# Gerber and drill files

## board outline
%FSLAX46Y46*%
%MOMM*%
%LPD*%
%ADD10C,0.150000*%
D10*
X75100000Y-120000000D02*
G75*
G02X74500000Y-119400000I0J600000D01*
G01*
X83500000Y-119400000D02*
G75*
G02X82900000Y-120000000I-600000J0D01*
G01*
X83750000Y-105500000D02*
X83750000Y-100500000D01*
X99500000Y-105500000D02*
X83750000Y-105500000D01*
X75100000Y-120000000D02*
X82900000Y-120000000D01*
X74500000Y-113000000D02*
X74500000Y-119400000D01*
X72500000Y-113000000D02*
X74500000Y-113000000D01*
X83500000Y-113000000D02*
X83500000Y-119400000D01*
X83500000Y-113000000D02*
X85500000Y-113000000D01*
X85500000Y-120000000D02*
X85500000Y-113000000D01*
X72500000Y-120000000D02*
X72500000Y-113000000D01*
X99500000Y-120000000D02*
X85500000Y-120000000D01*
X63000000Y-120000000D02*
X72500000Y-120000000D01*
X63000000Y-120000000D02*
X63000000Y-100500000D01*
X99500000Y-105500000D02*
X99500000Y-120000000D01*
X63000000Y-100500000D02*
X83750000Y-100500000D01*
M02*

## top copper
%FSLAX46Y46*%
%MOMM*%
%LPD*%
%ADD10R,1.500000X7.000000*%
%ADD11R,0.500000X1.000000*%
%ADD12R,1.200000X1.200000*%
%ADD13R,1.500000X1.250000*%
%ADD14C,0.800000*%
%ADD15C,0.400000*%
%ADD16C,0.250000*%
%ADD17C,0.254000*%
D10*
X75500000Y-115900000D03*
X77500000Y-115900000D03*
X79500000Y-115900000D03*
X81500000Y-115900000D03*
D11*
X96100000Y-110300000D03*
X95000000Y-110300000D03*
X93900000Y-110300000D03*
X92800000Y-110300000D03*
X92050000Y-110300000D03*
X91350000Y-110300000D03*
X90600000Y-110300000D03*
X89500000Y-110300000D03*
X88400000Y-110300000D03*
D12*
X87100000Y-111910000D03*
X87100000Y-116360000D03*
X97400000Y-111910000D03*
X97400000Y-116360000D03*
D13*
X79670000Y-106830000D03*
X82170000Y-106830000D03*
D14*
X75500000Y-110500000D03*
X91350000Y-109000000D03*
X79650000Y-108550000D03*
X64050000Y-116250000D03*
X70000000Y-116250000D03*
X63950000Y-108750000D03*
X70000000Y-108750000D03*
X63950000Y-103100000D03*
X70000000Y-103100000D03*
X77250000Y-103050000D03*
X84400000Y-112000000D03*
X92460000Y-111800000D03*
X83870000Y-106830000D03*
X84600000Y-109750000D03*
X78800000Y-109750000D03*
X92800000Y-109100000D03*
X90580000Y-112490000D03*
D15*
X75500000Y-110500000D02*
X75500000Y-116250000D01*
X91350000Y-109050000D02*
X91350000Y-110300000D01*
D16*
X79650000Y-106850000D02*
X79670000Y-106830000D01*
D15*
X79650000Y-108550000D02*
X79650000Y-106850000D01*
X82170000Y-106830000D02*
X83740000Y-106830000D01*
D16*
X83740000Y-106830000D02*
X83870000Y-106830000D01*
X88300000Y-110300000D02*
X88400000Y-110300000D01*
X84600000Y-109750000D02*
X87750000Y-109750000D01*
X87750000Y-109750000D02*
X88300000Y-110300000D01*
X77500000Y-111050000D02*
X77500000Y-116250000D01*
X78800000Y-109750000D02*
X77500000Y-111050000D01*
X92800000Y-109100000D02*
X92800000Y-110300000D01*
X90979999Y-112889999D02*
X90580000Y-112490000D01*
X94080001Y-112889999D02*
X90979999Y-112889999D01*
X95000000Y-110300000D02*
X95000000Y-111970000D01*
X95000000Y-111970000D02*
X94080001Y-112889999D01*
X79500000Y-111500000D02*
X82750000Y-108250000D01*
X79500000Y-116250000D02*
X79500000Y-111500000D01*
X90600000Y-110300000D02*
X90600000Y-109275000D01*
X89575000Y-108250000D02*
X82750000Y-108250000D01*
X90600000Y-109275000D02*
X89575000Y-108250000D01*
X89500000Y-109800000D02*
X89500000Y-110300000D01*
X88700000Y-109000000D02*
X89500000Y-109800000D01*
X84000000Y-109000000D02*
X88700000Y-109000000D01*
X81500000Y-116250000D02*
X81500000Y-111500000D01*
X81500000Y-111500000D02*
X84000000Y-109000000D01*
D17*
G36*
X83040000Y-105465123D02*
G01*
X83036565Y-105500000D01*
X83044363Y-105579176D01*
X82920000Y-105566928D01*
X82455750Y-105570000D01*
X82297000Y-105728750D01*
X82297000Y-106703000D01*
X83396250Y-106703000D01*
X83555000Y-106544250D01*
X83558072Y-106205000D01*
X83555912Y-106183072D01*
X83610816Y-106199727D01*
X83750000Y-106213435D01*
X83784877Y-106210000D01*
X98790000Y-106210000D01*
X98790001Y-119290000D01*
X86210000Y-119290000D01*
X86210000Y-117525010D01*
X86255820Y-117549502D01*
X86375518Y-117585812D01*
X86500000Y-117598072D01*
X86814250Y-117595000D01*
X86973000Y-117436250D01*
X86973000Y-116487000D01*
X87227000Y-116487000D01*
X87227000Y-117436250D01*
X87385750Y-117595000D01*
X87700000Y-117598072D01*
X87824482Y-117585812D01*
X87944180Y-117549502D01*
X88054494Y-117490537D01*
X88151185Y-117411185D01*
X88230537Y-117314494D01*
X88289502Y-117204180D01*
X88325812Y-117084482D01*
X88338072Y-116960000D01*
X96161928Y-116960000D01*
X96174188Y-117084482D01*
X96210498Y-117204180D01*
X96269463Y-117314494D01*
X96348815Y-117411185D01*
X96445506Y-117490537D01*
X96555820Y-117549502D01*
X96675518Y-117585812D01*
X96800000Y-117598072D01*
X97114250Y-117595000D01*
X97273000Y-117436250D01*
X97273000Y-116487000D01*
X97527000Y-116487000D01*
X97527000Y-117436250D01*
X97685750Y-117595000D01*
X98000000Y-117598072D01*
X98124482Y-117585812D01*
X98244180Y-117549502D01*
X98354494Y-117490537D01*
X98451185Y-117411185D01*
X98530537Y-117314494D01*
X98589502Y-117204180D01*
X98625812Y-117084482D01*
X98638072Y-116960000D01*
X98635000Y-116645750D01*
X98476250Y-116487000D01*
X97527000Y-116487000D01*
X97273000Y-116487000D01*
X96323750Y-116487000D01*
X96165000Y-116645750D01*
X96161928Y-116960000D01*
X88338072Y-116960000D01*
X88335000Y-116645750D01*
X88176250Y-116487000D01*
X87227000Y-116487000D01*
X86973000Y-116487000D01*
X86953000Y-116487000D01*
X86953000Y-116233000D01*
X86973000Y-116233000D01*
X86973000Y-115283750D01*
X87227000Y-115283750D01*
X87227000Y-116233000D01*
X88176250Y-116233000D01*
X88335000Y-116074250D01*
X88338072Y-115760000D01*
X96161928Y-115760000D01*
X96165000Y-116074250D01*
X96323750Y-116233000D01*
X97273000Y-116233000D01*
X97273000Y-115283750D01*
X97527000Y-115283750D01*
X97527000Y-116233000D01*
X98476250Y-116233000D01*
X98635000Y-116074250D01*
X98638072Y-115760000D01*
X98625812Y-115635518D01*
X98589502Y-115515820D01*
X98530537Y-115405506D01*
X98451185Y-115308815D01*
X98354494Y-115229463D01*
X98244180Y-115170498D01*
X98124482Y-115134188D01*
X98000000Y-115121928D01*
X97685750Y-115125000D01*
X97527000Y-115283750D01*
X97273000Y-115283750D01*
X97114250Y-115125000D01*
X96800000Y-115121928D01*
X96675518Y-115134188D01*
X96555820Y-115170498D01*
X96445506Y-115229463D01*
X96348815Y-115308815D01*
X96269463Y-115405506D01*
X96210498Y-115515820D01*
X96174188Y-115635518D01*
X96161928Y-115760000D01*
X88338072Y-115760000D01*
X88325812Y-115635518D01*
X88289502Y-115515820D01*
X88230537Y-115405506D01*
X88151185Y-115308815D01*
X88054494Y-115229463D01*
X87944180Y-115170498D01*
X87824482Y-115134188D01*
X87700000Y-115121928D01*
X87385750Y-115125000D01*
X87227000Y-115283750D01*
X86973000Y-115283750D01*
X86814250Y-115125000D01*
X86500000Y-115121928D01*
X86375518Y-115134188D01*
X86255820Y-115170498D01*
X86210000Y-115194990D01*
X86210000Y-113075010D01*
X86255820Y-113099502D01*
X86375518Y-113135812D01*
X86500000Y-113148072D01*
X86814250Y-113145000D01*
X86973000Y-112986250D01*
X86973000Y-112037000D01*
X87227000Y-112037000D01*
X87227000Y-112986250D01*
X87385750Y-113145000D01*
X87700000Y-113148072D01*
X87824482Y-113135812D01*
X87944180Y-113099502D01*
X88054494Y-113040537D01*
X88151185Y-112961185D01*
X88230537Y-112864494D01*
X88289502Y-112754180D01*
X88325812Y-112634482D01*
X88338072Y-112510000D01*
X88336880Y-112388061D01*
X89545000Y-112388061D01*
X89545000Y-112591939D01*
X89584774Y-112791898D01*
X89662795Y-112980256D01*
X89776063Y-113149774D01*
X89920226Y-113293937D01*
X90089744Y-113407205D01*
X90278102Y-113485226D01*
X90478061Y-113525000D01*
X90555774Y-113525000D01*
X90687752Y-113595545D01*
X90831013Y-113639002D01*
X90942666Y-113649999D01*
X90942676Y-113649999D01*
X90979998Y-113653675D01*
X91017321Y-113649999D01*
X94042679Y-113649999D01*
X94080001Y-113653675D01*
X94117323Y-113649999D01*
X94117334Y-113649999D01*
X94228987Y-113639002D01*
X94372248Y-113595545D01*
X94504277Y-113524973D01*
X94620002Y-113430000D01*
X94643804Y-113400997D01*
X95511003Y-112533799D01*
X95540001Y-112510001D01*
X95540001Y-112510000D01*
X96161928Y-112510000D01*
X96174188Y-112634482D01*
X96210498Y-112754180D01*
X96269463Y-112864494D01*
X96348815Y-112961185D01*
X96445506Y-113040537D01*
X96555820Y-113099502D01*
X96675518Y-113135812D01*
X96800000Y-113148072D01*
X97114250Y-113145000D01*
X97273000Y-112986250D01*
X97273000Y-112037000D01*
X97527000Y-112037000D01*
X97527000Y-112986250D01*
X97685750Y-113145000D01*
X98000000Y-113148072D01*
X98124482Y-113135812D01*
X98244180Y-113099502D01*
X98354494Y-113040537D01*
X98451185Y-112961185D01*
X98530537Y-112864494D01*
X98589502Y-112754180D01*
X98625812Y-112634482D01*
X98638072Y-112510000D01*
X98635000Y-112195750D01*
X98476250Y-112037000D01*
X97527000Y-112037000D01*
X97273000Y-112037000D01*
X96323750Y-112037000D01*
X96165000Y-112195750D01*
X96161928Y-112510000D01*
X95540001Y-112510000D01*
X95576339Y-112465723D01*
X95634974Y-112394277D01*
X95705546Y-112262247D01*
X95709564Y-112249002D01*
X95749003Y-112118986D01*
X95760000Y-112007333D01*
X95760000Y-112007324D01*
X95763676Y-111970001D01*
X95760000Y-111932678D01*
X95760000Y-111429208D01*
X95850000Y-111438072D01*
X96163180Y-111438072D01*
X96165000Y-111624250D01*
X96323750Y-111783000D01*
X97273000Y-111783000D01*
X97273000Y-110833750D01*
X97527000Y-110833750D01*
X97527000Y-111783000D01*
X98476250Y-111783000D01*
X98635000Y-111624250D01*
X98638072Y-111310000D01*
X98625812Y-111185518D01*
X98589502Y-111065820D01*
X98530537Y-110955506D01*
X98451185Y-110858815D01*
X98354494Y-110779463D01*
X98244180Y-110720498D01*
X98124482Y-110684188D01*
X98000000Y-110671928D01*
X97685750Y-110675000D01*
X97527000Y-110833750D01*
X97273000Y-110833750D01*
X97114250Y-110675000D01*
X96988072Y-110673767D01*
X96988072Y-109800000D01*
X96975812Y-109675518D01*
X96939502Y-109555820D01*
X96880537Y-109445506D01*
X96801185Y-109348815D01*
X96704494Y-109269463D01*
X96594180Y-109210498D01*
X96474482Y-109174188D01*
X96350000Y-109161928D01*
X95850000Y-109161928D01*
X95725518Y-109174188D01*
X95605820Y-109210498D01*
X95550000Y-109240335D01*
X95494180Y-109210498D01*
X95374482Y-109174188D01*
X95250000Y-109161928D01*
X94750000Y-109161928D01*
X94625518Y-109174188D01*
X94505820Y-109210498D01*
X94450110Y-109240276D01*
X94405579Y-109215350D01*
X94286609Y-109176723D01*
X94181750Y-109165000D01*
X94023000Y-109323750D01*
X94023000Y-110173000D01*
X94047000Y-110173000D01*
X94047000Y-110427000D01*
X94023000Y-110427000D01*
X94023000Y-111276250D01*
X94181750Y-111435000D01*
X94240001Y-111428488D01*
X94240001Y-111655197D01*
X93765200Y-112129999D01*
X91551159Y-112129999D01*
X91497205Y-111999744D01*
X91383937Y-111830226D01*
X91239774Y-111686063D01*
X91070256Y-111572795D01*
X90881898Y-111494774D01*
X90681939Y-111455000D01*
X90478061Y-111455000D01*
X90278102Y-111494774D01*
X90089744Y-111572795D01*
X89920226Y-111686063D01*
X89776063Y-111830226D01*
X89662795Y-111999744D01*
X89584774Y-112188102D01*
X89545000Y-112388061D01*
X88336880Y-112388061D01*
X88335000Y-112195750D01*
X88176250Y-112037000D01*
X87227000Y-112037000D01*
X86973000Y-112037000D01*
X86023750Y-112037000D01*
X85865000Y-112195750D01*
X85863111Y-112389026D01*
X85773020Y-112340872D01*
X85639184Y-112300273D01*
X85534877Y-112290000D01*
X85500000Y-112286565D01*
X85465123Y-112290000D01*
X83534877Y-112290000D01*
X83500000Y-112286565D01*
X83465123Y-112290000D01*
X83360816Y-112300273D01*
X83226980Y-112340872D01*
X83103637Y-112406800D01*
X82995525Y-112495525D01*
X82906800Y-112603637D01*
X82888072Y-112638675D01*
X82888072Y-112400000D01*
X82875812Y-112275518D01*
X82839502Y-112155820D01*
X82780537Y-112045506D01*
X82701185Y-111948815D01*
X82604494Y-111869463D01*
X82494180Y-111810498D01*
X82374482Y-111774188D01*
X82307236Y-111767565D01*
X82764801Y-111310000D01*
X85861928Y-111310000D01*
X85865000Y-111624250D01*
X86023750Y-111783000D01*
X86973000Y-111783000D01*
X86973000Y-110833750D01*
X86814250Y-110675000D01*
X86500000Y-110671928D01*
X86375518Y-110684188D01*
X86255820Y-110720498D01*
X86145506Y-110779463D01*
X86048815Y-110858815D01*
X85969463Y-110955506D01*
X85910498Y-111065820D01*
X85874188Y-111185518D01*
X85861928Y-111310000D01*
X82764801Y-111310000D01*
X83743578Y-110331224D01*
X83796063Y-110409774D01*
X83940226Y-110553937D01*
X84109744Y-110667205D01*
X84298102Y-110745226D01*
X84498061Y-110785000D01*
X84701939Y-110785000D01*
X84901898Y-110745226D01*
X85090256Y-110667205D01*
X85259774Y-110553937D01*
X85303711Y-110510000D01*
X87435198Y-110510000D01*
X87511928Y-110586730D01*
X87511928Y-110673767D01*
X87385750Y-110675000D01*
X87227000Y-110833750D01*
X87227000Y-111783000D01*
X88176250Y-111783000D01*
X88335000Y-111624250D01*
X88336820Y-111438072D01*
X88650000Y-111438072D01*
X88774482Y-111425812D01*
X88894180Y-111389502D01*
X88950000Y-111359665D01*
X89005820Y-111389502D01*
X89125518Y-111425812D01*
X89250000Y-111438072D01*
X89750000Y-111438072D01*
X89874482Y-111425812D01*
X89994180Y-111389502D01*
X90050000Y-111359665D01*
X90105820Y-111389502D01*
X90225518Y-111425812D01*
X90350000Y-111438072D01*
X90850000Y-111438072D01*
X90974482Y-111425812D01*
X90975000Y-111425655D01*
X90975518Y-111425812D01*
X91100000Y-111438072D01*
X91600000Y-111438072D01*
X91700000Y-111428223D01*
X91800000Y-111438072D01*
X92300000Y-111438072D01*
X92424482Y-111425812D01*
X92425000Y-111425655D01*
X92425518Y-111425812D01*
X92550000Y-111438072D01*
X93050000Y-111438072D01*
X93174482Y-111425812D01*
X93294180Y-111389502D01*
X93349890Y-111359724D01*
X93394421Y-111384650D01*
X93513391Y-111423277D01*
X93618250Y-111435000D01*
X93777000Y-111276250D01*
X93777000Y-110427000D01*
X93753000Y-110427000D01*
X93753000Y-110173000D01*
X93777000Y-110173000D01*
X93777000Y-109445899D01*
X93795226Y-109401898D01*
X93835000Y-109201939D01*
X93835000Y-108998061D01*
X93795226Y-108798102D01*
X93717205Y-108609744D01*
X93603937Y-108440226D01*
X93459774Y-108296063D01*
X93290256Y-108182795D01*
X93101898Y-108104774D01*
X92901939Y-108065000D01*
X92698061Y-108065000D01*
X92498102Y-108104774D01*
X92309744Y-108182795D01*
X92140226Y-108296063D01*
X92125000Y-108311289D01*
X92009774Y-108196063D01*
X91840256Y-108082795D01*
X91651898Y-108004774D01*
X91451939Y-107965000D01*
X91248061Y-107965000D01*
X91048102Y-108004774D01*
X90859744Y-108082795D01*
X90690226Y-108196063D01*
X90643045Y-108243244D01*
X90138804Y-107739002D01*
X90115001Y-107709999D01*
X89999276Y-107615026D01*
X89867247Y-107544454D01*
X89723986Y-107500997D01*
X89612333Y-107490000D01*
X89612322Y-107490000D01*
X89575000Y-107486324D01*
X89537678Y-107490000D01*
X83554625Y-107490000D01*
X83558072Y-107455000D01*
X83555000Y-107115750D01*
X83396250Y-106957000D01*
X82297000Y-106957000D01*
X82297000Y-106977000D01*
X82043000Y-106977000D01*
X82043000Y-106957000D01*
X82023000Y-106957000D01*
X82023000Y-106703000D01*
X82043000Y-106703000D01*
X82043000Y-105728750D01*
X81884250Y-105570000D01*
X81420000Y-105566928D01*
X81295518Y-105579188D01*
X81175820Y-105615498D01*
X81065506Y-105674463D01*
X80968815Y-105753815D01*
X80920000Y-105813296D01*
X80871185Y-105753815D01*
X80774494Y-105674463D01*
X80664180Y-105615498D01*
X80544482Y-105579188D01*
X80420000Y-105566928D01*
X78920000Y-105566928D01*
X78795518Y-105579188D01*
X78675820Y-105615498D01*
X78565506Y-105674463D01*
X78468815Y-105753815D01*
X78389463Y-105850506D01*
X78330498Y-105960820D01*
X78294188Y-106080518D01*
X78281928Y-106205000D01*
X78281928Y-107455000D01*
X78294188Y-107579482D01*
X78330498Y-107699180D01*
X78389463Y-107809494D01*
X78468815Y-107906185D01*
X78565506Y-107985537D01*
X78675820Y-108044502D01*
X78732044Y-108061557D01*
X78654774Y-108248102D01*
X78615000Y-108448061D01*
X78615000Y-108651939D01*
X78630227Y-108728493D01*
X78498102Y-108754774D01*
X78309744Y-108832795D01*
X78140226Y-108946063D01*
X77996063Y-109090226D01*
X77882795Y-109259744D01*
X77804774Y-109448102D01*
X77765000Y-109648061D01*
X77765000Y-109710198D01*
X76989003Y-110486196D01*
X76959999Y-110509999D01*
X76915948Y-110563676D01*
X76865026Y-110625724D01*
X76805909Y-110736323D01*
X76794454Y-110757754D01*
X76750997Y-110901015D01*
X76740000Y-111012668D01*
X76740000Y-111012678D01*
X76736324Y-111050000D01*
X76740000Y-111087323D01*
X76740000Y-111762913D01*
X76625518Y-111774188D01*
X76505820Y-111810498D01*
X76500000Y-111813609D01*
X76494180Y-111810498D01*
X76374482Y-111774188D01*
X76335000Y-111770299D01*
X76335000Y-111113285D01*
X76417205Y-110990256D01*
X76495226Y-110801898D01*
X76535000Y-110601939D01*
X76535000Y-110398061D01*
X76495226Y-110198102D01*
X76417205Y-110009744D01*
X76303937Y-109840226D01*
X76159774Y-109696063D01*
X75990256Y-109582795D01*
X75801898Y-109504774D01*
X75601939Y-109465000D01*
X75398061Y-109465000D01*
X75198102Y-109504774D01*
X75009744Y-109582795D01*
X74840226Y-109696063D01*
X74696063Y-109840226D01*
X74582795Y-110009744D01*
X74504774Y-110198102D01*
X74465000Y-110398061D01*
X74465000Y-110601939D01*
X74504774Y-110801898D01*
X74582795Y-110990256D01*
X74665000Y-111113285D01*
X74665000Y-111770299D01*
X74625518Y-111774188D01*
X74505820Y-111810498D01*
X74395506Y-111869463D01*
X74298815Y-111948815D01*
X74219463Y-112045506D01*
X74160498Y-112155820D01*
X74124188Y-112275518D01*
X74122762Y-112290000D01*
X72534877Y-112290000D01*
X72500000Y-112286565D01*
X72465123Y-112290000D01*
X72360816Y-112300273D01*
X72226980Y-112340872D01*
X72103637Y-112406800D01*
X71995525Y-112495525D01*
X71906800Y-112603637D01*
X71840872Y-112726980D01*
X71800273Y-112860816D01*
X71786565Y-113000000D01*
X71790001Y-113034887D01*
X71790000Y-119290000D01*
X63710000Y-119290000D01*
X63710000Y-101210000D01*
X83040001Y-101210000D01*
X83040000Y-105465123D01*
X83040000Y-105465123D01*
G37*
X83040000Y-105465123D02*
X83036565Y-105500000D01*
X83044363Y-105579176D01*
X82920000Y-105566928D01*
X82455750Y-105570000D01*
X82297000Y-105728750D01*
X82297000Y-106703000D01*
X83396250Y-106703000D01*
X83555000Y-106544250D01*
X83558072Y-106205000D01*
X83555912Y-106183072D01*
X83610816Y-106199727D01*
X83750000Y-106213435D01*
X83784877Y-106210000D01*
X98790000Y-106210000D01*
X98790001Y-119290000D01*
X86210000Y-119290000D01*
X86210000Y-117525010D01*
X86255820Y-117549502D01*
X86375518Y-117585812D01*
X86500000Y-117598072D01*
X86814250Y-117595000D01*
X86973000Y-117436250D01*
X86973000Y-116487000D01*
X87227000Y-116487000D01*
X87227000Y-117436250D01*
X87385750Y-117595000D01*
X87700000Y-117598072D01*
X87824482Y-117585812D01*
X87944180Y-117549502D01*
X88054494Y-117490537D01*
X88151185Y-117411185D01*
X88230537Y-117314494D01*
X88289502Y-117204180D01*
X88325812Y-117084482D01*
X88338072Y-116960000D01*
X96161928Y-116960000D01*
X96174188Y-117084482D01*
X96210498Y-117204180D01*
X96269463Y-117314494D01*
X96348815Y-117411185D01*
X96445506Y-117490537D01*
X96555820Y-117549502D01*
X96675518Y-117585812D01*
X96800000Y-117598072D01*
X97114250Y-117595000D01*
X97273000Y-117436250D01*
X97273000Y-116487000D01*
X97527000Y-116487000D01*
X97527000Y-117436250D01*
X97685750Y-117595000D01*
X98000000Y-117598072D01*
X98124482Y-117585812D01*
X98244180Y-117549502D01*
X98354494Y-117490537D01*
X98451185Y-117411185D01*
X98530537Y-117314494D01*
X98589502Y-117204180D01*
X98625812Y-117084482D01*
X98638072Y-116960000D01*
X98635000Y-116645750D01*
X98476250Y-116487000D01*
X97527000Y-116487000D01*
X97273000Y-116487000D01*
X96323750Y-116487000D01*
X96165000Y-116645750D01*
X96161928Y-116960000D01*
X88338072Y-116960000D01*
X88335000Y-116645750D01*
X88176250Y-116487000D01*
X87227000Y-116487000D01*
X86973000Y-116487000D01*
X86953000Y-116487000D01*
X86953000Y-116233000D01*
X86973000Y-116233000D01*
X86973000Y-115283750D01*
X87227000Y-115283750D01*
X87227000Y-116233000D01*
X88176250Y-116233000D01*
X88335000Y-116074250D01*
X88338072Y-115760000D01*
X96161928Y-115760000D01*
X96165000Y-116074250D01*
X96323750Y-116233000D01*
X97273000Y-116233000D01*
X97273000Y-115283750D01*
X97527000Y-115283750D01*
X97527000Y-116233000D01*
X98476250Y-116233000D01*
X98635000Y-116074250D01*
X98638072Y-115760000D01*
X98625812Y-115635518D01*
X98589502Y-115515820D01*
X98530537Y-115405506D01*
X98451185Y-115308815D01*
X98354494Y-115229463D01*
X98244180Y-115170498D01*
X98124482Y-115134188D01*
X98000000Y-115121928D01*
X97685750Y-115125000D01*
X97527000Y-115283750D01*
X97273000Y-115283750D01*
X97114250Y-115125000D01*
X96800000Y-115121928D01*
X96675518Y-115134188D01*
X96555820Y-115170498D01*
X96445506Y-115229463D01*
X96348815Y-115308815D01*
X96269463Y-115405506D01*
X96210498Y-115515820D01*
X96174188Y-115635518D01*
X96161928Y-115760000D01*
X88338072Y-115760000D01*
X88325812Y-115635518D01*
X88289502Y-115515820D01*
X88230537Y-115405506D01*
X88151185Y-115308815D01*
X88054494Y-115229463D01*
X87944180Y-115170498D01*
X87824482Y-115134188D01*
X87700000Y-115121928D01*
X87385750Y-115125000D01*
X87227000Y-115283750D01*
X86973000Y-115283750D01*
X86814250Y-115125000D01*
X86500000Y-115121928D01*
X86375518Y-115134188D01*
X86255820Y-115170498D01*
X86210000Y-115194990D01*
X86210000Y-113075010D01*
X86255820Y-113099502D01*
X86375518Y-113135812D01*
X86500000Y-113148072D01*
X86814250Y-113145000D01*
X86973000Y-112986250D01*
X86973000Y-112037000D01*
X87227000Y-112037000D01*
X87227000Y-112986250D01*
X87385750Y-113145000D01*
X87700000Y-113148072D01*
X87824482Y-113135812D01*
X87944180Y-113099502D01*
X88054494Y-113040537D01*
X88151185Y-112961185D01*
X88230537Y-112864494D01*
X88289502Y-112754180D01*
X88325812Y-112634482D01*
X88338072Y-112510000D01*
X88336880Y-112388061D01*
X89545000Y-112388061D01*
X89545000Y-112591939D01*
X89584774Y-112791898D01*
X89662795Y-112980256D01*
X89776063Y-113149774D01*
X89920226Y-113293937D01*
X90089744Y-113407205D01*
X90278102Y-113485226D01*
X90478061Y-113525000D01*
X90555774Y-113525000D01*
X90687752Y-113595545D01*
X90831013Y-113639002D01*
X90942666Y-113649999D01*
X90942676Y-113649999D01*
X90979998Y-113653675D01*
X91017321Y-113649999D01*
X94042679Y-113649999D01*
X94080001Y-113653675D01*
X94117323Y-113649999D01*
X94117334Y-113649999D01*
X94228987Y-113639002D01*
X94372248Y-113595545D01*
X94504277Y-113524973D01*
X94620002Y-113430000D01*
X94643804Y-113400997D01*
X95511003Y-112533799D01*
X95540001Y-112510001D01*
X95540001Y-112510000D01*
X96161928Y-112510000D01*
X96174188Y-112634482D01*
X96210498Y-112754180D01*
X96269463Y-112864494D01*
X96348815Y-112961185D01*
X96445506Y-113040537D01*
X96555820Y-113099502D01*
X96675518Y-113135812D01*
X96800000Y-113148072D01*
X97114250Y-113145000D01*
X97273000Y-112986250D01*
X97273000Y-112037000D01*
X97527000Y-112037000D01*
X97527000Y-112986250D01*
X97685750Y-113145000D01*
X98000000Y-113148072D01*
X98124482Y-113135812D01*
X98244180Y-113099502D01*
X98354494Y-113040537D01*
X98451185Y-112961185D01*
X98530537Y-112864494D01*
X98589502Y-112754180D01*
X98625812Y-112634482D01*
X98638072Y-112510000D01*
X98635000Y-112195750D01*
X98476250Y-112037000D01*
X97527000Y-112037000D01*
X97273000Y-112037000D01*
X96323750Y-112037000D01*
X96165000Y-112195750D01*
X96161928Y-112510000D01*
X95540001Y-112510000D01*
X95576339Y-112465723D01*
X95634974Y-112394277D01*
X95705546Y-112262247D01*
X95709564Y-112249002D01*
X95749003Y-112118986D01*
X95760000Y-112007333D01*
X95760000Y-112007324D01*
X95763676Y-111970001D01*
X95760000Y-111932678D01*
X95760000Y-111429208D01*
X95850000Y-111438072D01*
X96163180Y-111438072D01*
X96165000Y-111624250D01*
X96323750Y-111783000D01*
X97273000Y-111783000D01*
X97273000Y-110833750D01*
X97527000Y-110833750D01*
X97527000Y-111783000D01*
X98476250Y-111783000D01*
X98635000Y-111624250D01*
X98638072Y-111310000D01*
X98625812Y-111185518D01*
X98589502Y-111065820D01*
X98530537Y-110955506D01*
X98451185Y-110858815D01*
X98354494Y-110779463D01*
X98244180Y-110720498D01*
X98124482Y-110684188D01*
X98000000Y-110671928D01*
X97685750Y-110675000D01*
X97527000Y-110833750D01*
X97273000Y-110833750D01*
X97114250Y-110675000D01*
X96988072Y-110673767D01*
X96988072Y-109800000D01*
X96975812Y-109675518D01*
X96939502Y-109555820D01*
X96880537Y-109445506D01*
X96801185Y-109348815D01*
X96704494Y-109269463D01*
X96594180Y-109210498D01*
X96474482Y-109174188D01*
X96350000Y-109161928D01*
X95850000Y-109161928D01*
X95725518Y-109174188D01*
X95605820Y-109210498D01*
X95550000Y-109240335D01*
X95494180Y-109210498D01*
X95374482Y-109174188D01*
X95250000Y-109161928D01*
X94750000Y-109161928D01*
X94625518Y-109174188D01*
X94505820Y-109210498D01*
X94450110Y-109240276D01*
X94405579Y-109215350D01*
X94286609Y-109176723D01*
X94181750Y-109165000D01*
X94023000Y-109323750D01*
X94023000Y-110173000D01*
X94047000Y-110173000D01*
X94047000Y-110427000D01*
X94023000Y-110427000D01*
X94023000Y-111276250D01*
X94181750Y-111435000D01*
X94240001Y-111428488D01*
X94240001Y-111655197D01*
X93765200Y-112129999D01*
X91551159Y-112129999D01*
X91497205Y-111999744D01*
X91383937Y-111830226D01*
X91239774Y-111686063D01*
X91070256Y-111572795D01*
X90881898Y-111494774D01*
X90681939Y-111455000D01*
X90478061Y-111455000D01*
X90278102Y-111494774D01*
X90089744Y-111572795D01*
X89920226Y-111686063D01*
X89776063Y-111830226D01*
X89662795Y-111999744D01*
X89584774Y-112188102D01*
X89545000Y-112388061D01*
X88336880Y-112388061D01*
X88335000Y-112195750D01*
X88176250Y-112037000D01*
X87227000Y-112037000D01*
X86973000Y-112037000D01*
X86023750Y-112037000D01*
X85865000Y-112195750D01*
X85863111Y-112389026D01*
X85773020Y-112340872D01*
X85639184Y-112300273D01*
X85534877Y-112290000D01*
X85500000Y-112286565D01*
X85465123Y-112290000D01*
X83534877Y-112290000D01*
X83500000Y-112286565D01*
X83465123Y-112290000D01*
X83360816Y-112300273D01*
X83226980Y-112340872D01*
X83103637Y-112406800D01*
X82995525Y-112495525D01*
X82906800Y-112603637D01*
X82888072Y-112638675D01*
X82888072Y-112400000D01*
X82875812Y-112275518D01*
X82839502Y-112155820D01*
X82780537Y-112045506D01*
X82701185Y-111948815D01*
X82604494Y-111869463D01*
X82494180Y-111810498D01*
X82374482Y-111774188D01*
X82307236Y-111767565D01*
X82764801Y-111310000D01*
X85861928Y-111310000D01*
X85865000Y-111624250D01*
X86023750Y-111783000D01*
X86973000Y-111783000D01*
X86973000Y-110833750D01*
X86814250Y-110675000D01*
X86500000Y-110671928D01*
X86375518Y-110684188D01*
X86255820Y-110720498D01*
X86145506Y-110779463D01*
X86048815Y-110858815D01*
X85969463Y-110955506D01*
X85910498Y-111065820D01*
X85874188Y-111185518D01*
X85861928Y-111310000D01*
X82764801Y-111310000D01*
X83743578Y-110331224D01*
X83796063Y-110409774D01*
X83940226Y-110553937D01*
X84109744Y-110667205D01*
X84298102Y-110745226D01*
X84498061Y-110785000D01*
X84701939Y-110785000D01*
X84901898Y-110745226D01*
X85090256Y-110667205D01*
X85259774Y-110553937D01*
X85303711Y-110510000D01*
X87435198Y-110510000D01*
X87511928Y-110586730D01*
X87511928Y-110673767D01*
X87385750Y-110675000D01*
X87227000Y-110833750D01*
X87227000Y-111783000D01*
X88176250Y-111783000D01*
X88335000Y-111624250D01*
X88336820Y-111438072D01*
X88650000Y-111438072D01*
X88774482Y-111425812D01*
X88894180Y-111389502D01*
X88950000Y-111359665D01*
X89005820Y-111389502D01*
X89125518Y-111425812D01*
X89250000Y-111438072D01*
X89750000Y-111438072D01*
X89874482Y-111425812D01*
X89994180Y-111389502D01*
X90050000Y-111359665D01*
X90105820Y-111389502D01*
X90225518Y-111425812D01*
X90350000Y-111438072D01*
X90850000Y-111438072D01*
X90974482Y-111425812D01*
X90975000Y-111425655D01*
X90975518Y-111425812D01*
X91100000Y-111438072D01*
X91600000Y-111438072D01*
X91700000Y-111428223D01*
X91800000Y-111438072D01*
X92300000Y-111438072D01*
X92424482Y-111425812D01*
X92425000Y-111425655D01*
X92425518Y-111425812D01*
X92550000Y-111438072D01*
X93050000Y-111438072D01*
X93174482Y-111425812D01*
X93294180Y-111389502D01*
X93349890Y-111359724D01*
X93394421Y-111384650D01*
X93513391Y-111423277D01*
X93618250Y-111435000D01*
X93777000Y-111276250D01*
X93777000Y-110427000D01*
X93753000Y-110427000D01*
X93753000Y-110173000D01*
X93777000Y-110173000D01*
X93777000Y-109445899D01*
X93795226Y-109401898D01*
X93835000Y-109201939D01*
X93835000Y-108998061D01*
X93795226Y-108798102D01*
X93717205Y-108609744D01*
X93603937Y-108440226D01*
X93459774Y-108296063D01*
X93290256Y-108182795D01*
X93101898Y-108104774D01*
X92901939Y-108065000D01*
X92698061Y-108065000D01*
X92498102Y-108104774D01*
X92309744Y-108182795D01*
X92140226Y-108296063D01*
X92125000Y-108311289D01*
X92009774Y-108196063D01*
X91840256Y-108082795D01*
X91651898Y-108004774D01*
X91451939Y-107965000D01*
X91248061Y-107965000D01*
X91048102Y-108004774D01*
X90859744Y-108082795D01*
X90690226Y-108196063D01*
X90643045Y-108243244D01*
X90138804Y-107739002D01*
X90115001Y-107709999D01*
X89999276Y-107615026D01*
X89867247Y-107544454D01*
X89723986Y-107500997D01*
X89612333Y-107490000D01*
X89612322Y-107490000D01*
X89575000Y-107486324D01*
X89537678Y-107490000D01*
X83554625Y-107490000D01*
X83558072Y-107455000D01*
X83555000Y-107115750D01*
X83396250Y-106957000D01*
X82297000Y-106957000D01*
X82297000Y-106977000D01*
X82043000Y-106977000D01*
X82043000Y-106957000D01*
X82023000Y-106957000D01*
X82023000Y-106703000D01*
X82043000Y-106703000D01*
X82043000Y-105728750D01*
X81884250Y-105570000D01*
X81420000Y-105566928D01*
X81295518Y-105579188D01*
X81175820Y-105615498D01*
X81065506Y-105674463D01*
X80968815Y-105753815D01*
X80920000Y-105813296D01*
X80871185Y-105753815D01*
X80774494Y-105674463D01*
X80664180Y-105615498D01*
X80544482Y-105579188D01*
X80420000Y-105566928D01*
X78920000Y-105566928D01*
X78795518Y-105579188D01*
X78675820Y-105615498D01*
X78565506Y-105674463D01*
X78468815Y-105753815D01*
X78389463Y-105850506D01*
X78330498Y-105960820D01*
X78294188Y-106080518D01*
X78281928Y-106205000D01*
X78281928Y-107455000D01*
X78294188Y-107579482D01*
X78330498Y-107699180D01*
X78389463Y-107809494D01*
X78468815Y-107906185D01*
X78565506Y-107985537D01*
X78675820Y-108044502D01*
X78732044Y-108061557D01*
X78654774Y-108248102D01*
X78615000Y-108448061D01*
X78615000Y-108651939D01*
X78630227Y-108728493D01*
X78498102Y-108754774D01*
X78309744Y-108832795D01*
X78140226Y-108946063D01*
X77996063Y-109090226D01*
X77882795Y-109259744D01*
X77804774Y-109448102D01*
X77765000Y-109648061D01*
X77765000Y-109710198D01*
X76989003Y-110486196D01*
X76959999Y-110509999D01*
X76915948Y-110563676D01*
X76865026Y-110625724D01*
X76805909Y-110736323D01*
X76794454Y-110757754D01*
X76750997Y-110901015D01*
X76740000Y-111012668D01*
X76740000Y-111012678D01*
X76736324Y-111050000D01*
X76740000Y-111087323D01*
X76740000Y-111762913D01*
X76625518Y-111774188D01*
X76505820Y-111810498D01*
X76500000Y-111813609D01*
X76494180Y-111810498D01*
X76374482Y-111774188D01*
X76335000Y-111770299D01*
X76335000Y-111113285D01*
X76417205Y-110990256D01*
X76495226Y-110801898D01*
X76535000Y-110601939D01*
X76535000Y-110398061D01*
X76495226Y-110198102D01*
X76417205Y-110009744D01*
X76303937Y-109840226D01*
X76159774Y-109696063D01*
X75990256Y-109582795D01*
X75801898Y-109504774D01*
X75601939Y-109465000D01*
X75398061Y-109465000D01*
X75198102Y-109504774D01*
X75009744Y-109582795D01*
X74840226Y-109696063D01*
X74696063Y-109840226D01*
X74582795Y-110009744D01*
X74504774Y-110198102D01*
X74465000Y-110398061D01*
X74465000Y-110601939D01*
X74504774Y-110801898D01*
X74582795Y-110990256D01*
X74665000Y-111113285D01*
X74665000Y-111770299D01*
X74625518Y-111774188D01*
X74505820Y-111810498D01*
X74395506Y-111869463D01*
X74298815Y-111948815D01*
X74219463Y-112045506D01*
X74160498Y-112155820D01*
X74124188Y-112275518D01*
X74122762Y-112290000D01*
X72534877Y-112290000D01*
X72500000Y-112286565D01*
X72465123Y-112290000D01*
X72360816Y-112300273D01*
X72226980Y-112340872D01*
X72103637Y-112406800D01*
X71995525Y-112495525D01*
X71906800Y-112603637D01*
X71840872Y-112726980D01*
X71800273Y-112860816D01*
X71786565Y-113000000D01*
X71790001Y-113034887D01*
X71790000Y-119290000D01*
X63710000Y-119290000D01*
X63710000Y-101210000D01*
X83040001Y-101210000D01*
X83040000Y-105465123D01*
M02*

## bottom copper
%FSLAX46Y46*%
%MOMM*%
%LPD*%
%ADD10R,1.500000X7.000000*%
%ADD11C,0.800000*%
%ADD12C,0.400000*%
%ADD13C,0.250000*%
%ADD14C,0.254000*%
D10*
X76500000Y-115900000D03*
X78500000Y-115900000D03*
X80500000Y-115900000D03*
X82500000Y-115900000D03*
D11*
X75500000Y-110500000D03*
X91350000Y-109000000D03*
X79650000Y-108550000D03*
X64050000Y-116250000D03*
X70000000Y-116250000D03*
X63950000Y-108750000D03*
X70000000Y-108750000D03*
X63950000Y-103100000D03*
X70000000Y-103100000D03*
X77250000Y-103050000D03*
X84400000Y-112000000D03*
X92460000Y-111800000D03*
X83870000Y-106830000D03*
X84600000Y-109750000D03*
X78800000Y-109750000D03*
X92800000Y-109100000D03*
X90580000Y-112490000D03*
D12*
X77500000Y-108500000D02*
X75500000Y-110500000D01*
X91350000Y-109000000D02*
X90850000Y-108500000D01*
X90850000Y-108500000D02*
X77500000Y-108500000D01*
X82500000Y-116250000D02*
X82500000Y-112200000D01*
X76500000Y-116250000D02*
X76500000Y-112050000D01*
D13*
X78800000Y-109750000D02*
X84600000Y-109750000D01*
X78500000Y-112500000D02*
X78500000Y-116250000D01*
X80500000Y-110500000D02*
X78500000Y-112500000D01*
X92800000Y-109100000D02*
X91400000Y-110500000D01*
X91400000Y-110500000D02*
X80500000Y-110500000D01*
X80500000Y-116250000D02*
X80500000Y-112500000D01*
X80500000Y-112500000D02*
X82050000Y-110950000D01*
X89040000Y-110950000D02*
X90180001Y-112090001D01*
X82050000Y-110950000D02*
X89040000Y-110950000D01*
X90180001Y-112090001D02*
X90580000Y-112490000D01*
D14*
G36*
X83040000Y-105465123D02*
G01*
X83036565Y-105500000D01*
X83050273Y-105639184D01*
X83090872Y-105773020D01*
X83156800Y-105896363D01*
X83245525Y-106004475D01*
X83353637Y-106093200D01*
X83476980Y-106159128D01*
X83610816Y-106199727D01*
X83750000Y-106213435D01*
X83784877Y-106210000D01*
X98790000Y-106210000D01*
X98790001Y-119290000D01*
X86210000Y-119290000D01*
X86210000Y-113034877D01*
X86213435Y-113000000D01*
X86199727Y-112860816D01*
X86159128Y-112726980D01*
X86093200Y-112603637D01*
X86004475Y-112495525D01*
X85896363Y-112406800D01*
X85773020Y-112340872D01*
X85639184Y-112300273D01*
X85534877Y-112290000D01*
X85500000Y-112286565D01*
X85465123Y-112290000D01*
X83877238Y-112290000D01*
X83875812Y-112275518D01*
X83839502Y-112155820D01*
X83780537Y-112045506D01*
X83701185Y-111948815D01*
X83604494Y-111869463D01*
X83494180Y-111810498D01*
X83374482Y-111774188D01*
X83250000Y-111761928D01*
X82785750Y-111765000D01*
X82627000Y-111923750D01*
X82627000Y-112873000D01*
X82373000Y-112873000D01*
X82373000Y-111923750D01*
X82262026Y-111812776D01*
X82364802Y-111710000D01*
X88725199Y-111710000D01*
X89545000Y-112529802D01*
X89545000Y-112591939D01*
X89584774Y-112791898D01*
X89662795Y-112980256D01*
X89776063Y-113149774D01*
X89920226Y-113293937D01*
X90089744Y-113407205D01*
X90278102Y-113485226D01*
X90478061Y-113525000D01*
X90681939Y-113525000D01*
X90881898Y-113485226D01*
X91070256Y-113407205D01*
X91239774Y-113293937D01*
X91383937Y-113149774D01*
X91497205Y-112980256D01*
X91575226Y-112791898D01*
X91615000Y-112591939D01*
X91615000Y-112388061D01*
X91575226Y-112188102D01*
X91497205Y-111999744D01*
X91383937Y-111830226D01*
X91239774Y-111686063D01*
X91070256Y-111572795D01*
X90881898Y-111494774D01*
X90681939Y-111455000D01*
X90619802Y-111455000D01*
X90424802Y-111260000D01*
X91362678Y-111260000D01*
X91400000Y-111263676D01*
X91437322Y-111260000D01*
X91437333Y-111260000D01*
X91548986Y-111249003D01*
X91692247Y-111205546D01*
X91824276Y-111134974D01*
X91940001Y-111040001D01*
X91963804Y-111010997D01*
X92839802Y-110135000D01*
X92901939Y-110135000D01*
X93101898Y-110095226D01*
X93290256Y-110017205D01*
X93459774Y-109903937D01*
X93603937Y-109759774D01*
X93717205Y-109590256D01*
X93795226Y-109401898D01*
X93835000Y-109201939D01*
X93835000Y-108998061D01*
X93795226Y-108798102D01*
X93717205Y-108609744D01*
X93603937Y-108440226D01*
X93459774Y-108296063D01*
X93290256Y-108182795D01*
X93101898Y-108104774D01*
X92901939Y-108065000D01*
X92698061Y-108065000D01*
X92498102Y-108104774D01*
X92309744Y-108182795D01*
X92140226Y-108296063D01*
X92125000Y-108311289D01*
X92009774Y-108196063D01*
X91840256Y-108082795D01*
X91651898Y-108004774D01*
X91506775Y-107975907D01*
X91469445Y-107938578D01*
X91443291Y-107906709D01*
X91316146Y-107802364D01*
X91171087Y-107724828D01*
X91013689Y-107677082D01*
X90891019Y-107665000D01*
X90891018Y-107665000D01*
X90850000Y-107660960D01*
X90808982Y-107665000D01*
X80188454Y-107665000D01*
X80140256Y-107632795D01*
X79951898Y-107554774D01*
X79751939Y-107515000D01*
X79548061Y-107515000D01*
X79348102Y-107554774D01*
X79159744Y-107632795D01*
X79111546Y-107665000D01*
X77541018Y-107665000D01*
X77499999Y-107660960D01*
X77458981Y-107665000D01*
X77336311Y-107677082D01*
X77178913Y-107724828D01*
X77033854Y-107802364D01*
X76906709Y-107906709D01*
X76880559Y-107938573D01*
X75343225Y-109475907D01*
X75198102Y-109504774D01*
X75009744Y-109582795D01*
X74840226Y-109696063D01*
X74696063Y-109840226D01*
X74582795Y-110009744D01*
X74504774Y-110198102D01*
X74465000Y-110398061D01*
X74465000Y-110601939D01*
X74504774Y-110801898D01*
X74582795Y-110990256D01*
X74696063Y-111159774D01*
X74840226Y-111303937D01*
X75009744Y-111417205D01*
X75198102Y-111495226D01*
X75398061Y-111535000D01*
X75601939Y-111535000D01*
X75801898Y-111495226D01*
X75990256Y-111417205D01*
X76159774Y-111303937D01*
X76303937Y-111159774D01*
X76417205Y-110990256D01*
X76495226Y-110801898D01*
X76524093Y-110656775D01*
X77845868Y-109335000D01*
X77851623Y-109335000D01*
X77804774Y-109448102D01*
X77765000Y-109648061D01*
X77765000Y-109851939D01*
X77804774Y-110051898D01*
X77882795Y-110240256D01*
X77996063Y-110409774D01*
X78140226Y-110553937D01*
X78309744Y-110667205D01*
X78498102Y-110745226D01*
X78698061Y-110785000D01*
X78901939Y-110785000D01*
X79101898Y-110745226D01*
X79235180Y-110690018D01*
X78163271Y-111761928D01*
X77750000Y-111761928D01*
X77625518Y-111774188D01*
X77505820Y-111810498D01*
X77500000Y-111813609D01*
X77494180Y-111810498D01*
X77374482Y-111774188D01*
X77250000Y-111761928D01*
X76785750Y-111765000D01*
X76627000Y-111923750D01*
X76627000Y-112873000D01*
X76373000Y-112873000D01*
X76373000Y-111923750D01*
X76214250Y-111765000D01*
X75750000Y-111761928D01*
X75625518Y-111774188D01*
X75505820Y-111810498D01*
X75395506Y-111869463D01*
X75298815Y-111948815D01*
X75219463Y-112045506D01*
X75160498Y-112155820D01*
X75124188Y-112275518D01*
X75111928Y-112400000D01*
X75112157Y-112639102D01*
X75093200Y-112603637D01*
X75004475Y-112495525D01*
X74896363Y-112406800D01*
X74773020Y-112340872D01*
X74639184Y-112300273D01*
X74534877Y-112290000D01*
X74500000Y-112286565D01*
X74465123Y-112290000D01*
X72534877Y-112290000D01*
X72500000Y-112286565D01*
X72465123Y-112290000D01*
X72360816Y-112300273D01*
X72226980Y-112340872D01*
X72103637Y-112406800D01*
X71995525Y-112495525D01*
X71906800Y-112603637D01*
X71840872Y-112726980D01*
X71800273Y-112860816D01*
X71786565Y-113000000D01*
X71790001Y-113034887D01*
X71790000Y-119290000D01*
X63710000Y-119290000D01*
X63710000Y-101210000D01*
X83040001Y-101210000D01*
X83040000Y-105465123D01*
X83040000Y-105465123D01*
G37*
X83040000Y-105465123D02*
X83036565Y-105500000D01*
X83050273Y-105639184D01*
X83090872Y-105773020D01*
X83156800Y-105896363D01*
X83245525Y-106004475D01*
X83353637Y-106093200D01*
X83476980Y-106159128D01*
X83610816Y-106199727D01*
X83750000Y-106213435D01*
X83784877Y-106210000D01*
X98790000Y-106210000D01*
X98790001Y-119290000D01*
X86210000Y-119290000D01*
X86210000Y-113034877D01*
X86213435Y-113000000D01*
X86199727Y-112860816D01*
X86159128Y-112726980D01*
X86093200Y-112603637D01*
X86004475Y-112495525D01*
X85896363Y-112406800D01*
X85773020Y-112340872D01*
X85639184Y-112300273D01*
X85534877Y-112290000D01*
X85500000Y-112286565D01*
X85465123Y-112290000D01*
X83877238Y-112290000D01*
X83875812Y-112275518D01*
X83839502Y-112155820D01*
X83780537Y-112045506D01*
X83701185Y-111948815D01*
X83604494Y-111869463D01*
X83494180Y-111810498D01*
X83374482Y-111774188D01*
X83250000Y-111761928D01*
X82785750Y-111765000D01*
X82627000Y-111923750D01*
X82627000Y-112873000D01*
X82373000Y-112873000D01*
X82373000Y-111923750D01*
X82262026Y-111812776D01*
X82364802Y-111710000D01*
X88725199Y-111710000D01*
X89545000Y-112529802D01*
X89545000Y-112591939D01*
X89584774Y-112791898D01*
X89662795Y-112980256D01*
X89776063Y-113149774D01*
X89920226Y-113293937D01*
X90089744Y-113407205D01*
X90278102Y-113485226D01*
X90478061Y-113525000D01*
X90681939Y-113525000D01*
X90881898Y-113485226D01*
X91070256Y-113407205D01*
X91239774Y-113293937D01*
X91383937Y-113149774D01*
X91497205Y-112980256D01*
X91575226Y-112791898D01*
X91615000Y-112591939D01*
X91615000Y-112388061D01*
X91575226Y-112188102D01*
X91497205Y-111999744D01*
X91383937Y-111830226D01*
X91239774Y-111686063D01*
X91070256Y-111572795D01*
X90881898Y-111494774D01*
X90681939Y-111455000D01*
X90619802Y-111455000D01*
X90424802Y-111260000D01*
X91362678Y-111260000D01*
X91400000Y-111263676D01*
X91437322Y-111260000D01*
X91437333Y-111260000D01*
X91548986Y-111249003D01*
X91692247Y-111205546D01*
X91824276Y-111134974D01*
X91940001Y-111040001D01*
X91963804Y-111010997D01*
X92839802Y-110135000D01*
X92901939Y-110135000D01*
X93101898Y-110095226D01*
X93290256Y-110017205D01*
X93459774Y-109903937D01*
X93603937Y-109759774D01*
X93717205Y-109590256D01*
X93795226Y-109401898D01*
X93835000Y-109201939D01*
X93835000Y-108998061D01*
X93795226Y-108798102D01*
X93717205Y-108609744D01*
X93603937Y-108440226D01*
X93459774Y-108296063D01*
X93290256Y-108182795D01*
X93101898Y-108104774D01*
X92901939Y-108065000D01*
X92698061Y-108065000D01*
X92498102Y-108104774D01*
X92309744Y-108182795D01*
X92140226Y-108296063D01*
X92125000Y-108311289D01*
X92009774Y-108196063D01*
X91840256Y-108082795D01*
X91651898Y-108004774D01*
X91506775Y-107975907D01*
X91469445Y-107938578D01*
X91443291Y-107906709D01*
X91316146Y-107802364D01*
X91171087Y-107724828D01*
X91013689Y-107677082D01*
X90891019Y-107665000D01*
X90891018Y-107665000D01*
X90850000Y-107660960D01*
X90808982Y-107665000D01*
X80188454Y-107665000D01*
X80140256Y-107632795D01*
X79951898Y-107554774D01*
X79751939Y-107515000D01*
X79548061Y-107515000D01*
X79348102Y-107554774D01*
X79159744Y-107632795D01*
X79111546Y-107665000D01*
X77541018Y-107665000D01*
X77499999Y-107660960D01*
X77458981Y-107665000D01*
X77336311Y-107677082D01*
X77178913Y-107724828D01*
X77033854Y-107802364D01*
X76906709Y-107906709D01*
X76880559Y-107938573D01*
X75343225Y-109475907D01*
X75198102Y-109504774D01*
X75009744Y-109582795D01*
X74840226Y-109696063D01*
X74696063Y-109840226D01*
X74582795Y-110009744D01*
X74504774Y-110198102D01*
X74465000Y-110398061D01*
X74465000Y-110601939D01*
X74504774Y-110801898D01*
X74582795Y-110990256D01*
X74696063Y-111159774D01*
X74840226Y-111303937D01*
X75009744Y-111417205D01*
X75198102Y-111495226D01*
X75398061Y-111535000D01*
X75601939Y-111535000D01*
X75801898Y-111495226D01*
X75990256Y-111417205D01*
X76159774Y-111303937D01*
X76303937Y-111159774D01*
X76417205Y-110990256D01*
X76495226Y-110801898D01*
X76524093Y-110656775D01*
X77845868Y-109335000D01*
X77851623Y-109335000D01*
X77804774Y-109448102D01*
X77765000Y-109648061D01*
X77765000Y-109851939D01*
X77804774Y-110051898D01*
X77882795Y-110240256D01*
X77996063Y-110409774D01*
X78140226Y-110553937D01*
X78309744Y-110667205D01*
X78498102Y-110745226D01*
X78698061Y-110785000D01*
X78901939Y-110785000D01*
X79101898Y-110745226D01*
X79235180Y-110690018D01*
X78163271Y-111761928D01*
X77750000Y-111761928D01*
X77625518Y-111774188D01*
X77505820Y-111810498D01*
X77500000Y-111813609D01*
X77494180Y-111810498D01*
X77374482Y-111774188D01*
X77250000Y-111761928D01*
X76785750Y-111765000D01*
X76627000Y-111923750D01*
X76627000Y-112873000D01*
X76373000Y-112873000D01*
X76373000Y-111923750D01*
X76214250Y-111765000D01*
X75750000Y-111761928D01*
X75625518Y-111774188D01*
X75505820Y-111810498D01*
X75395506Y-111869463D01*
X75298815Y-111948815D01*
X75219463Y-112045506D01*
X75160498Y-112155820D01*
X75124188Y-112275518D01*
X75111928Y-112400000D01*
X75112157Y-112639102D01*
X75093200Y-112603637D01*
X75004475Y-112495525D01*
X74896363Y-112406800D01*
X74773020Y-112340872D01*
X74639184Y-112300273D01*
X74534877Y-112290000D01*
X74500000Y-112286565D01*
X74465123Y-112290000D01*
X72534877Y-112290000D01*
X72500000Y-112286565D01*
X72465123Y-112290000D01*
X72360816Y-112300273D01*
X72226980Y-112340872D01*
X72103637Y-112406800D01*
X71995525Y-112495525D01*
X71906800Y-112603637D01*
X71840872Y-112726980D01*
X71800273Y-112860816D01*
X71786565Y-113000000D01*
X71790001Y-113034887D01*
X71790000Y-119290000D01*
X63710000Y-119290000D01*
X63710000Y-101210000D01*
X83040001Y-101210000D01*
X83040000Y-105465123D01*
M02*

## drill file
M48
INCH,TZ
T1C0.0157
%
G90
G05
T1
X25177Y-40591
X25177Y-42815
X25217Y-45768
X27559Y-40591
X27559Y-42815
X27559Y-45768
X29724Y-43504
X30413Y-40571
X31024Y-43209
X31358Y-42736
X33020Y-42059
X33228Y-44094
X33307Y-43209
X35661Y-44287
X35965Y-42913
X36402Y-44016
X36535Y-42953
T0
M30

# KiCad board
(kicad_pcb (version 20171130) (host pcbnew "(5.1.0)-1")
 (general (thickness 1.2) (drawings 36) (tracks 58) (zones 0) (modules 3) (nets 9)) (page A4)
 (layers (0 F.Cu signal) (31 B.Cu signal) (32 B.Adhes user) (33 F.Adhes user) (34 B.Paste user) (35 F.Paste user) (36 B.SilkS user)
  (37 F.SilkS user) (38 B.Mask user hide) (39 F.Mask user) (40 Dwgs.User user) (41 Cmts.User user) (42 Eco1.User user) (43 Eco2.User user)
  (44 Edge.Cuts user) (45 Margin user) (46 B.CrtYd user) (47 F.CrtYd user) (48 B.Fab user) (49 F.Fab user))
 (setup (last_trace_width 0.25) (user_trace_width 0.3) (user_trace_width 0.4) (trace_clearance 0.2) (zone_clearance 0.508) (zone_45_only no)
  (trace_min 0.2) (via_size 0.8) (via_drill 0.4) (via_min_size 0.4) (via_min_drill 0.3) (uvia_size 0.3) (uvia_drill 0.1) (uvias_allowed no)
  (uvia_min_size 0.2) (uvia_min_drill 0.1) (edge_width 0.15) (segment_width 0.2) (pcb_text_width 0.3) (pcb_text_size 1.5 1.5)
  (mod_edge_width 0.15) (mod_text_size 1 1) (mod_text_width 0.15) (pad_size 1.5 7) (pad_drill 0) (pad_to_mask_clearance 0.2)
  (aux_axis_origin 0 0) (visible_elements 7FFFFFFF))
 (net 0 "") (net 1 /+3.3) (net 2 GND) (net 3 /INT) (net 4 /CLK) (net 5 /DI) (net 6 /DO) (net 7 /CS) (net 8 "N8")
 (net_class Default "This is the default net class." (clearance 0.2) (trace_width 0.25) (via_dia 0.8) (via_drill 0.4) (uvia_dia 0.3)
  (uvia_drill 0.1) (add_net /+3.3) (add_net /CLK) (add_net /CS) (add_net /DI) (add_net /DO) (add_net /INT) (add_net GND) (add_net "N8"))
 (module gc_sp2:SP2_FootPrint (layer F.Cu) (at 75.5 115.9)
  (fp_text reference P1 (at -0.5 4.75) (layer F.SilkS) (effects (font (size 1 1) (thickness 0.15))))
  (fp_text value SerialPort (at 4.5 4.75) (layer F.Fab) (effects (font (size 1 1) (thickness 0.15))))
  (pad 1 smd rect (at 0 0) (size 1.5 7) (layers F.Cu F.Paste F.Mask) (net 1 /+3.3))
  (pad 2 smd rect (at 1 0) (size 1.5 7) (layers B.Cu B.Paste B.Mask) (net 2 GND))
  (pad 3 smd rect (at 2 0) (size 1.5 7) (layers F.Cu F.Paste F.Mask) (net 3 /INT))
  (pad 4 smd rect (at 3 0) (size 1.5 7) (layers B.Cu B.Adhes B.Mask) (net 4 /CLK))
  (pad 5 smd rect (at 4 0) (size 1.5 7) (layers F.Cu F.Paste F.Mask) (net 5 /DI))
  (pad 6 smd rect (at 5 0) (size 1.5 7) (layers B.Cu B.Paste B.Mask) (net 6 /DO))
  (pad 7 smd rect (at 6 0) (size 1.5 7) (layers F.Cu F.Paste F.Mask) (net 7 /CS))
  (pad 8 smd rect (at 7 0) (size 1.5 7) (layers B.Cu B.Paste B.Mask) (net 2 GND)))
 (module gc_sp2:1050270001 (layer F.Cu) (at 96.1 110.3 180)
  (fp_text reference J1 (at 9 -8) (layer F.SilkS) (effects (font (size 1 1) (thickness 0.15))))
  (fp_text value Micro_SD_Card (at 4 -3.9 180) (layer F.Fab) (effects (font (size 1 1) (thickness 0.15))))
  (pad 8 smd rect (at 0 0 180) (size 0.5 1) (layers F.Cu F.Paste F.Mask) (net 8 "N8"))
  (pad 7 smd rect (at 1.1 0 180) (size 0.5 1) (layers F.Cu F.Paste F.Mask) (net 6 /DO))
  (pad 6 smd rect (at 2.2 0 180) (size 0.5 1) (layers F.Cu F.Paste F.Mask) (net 2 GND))
  (pad 5 smd rect (at 3.3 0 180) (size 0.5 1) (layers F.Cu F.Paste F.Mask) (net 4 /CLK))
  (pad "" smd rect (at 4.05 0 180) (size 0.5 1) (layers F.Cu F.Paste F.Mask))
  (pad 4 smd rect (at 4.75 0 180) (size 0.5 1) (layers F.Cu F.Paste F.Mask) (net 1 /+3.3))
  (pad 3 smd rect (at 5.5 0 180) (size 0.5 1) (layers F.Cu F.Paste F.Mask) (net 5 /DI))
  (pad 2 smd rect (at 6.6 0 180) (size 0.5 1) (layers F.Cu F.Paste F.Mask) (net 7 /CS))
  (pad 1 smd rect (at 7.7 0 180) (size 0.5 1) (layers F.Cu F.Paste F.Mask) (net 3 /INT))
  (pad 9 smd rect (at 9 -1.61 180) (size 1.2 1.2) (layers F.Cu F.Paste F.Mask) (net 2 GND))
  (pad 9 smd rect (at 9 -6.06 180) (size 1.2 1.2) (layers F.Cu F.Paste F.Mask) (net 2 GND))
  (pad 9 smd rect (at -1.3 -1.61 180) (size 1.2 1.2) (layers F.Cu F.Paste F.Mask) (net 2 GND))
  (pad 9 smd rect (at -1.3 -6.06 180) (size 1.2 1.2) (layers F.Cu F.Paste F.Mask) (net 2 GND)))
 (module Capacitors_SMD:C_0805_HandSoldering (layer F.Cu) (at 80.92 106.83)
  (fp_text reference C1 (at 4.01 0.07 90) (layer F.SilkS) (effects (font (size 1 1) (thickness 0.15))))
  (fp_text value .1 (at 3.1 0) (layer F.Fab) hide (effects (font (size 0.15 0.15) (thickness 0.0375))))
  (pad 1 smd rect (at -1.25 0) (size 1.5 1.25) (layers F.Cu F.Paste F.Mask) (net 1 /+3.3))
  (pad 2 smd rect (at 1.25 0) (size 1.5 1.25) (layers F.Cu F.Paste F.Mask) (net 2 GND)))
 (gr_arc (start 75.1 119.4) (end 74.5 119.4) (angle -90) (layer Edge.Cuts) (width 0.15))
 (gr_arc (start 82.9 119.4) (end 82.9 120) (angle -90) (layer Edge.Cuts) (width 0.15))
 (gr_line (start 83.75 105.5) (end 83.75 100.5) (layer Edge.Cuts) (width 0.15))
 (gr_line (start 99.5 105.5) (end 83.75 105.5) (layer Edge.Cuts) (width 0.15))
 (gr_line (start 75.1 120) (end 82.9 120) (layer Edge.Cuts) (width 0.15))
 (gr_line (start 74.5 113) (end 74.5 119.4) (layer Edge.Cuts) (width 0.15))
 (gr_line (start 72.5 113) (end 74.5 113) (layer Edge.Cuts) (width 0.15))
 (gr_line (start 83.5 113) (end 83.5 119.4) (layer Edge.Cuts) (width 0.15))
 (gr_line (start 83.5 113) (end 85.5 113) (layer Edge.Cuts) (width 0.15))
 (gr_line (start 85.5 120) (end 85.5 113) (layer Edge.Cuts) (width 0.15))
 (gr_line (start 72.5 120) (end 72.5 113) (layer Edge.Cuts) (width 0.15))
 (gr_line (start 99.5 120) (end 85.5 120) (layer Edge.Cuts) (width 0.15))
 (gr_line (start 63 120) (end 72.5 120) (layer Edge.Cuts) (width 0.15))
 (gr_line (start 63 120) (end 63 100.5) (layer Edge.Cuts) (width 0.15))
 (gr_line (start 99.5 105.5) (end 99.5 120) (layer Edge.Cuts) (width 0.15))
 (gr_line (start 63 100.5) (end 83.75 100.5) (layer Edge.Cuts) (width 0.15))
 (via (at 75.5 110.5) (size 0.8) (drill 0.4) (layers F.Cu B.Cu) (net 1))
 (segment (start 75.5 110.5) (end 75.5 116.25) (width 0.4) (layer F.Cu) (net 1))
 (segment (start 91.35 109.05) (end 91.35 110.3) (width 0.4) (layer F.Cu) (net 1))
 (via (at 91.35 109) (size 0.8) (drill 0.4) (layers F.Cu B.Cu) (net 1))
 (segment (start 77.5 108.5) (end 75.5 110.5) (width 0.4) (layer B.Cu) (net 1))
 (segment (start 91.35 109) (end 90.85 108.5) (width 0.4) (layer B.Cu) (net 1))
 (segment (start 90.85 108.5) (end 77.5 108.5) (width 0.4) (layer B.Cu) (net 1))
 (via (at 79.65 108.55) (size 0.8) (drill 0.4) (layers F.Cu B.Cu) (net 1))
 (segment (start 79.65 106.85) (end 79.67 106.83) (width 0.25) (layer F.Cu) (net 1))
 (segment (start 79.65 108.55) (end 79.65 106.85) (width 0.4) (layer F.Cu) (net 1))
 (via (at 64.05 116.25) (size 0.8) (drill 0.4) (layers F.Cu B.Cu) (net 2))
 (via (at 70 116.25) (size 0.8) (drill 0.4) (layers F.Cu B.Cu) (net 2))
 (via (at 63.95 108.75) (size 0.8) (drill 0.4) (layers F.Cu B.Cu) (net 2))
 (via (at 70 108.75) (size 0.8) (drill 0.4) (layers F.Cu B.Cu) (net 2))
 (via (at 63.95 103.1) (size 0.8) (drill 0.4) (layers F.Cu B.Cu) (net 2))
 (via (at 70 103.1) (size 0.8) (drill 0.4) (layers F.Cu B.Cu) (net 2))
 (via (at 77.25 103.05) (size 0.8) (drill 0.4) (layers F.Cu B.Cu) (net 2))
 (via (at 84.4 112) (size 0.8) (drill 0.4) (layers F.Cu B.Cu) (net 2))
 (segment (start 82.5 116.25) (end 82.5 112.2) (width 0.4) (layer B.Cu) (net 2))
 (segment (start 76.5 116.25) (end 76.5 112.05) (width 0.4) (layer B.Cu) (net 2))
 (via (at 92.46 111.8) (size 0.8) (drill 0.4) (layers F.Cu B.Cu) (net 2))
 (segment (start 82.17 106.83) (end 83.74 106.83) (width 0.4) (layer F.Cu) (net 2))
 (via (at 83.87 106.83) (size 0.8) (drill 0.4) (layers F.Cu B.Cu) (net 2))
 (segment (start 83.74 106.83) (end 83.87 106.83) (width 0.25) (layer F.Cu) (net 2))
 (via (at 84.6 109.75) (size 0.8) (drill 0.4) (layers F.Cu B.Cu) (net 3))
 (segment (start 88.3 110.3) (end 88.4 110.3) (width 0.25) (layer F.Cu) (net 3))
 (segment (start 84.6 109.75) (end 87.75 109.75) (width 0.25) (layer F.Cu) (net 3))
 (segment (start 87.75 109.75) (end 88.3 110.3) (width 0.25) (layer F.Cu) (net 3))
 (via (at 78.8 109.75) (size 0.8) (drill 0.4) (layers F.Cu B.Cu) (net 3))
 (segment (start 78.8 109.75) (end 84.6 109.75) (width 0.25) (layer B.Cu) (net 3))
 (segment (start 77.5 111.05) (end 77.5 116.25) (width 0.25) (layer F.Cu) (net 3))
 (segment (start 78.8 109.75) (end 77.5 111.05) (width 0.25) (layer F.Cu) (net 3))
 (via (at 92.8 109.1) (size 0.8) (drill 0.4) (layers F.Cu B.Cu) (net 4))
 (segment (start 92.8 109.1) (end 92.8 110.3) (width 0.25) (layer F.Cu) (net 4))
 (segment (start 78.5 112.5) (end 78.5 116.25) (width 0.25) (layer B.Cu) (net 4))
 (segment (start 80.5 110.5) (end 78.5 112.5) (width 0.25) (layer B.Cu) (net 4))
 (segment (start 92.8 109.1) (end 91.4 110.5) (width 0.25) (layer B.Cu) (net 4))
 (segment (start 91.4 110.5) (end 80.5 110.5) (width 0.25) (layer B.Cu) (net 4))
 (segment (start 80.5 116.25) (end 80.5 112.5) (width 0.25) (layer B.Cu) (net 6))
 (via (at 90.58 112.49) (size 0.8) (drill 0.4) (layers F.Cu B.Cu) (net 6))
 (segment (start 80.5 112.5) (end 82.05 110.95) (width 0.25) (layer B.Cu) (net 6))
 (segment (start 89.04 110.95) (end 90.180001 112.090001) (width 0.25) (layer B.Cu) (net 6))
 (segment (start 82.05 110.95) (end 89.04 110.95) (width 0.25) (layer B.Cu) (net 6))
 (segment (start 90.180001 112.090001) (end 90.58 112.49) (width 0.25) (layer B.Cu) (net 6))
 (segment (start 90.979999 112.889999) (end 90.58 112.49) (width 0.25) (layer F.Cu) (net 6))
 (segment (start 94.080001 112.889999) (end 90.979999 112.889999) (width 0.25) (layer F.Cu) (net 6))
 (segment (start 95 110.3) (end 95 111.97) (width 0.25) (layer F.Cu) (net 6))
 (segment (start 95 111.97) (end 94.080001 112.889999) (width 0.25) (layer F.Cu) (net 6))
 (segment (start 79.5 111.5) (end 82.75 108.25) (width 0.25) (layer F.Cu) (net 5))
 (segment (start 79.5 116.25) (end 79.5 111.5) (width 0.25) (layer F.Cu) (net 5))
 (segment (start 90.6 110.3) (end 90.6 109.275) (width 0.25) (layer F.Cu) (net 5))
 (segment (start 89.575 108.25) (end 82.75 108.25) (width 0.25) (layer F.Cu) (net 5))
 (segment (start 90.6 109.275) (end 89.575 108.25) (width 0.25) (layer F.Cu) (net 5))
 (segment (start 89.5 109.8) (end 89.5 110.3) (width 0.25) (layer F.Cu) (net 7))
 (segment (start 88.7 109) (end 89.5 109.8) (width 0.25) (layer F.Cu) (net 7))
 (segment (start 84 109) (end 88.7 109) (width 0.25) (layer F.Cu) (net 7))
 (segment (start 81.5 116.25) (end 81.5 111.5) (width 0.25) (layer F.Cu) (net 7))
 (segment (start 81.5 111.5) (end 84 109) (width 0.25) (layer F.Cu) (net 7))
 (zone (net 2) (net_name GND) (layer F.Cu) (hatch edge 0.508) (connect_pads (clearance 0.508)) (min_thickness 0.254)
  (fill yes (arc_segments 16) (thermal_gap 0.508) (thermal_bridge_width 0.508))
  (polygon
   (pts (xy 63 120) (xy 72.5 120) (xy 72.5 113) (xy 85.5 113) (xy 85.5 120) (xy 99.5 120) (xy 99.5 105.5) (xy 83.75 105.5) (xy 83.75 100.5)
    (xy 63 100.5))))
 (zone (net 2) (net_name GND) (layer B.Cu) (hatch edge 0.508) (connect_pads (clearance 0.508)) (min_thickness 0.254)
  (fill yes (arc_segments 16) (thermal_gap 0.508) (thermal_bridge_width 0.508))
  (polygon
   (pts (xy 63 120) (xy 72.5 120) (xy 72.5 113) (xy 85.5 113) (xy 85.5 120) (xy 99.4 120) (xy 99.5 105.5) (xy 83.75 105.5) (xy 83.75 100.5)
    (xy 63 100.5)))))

